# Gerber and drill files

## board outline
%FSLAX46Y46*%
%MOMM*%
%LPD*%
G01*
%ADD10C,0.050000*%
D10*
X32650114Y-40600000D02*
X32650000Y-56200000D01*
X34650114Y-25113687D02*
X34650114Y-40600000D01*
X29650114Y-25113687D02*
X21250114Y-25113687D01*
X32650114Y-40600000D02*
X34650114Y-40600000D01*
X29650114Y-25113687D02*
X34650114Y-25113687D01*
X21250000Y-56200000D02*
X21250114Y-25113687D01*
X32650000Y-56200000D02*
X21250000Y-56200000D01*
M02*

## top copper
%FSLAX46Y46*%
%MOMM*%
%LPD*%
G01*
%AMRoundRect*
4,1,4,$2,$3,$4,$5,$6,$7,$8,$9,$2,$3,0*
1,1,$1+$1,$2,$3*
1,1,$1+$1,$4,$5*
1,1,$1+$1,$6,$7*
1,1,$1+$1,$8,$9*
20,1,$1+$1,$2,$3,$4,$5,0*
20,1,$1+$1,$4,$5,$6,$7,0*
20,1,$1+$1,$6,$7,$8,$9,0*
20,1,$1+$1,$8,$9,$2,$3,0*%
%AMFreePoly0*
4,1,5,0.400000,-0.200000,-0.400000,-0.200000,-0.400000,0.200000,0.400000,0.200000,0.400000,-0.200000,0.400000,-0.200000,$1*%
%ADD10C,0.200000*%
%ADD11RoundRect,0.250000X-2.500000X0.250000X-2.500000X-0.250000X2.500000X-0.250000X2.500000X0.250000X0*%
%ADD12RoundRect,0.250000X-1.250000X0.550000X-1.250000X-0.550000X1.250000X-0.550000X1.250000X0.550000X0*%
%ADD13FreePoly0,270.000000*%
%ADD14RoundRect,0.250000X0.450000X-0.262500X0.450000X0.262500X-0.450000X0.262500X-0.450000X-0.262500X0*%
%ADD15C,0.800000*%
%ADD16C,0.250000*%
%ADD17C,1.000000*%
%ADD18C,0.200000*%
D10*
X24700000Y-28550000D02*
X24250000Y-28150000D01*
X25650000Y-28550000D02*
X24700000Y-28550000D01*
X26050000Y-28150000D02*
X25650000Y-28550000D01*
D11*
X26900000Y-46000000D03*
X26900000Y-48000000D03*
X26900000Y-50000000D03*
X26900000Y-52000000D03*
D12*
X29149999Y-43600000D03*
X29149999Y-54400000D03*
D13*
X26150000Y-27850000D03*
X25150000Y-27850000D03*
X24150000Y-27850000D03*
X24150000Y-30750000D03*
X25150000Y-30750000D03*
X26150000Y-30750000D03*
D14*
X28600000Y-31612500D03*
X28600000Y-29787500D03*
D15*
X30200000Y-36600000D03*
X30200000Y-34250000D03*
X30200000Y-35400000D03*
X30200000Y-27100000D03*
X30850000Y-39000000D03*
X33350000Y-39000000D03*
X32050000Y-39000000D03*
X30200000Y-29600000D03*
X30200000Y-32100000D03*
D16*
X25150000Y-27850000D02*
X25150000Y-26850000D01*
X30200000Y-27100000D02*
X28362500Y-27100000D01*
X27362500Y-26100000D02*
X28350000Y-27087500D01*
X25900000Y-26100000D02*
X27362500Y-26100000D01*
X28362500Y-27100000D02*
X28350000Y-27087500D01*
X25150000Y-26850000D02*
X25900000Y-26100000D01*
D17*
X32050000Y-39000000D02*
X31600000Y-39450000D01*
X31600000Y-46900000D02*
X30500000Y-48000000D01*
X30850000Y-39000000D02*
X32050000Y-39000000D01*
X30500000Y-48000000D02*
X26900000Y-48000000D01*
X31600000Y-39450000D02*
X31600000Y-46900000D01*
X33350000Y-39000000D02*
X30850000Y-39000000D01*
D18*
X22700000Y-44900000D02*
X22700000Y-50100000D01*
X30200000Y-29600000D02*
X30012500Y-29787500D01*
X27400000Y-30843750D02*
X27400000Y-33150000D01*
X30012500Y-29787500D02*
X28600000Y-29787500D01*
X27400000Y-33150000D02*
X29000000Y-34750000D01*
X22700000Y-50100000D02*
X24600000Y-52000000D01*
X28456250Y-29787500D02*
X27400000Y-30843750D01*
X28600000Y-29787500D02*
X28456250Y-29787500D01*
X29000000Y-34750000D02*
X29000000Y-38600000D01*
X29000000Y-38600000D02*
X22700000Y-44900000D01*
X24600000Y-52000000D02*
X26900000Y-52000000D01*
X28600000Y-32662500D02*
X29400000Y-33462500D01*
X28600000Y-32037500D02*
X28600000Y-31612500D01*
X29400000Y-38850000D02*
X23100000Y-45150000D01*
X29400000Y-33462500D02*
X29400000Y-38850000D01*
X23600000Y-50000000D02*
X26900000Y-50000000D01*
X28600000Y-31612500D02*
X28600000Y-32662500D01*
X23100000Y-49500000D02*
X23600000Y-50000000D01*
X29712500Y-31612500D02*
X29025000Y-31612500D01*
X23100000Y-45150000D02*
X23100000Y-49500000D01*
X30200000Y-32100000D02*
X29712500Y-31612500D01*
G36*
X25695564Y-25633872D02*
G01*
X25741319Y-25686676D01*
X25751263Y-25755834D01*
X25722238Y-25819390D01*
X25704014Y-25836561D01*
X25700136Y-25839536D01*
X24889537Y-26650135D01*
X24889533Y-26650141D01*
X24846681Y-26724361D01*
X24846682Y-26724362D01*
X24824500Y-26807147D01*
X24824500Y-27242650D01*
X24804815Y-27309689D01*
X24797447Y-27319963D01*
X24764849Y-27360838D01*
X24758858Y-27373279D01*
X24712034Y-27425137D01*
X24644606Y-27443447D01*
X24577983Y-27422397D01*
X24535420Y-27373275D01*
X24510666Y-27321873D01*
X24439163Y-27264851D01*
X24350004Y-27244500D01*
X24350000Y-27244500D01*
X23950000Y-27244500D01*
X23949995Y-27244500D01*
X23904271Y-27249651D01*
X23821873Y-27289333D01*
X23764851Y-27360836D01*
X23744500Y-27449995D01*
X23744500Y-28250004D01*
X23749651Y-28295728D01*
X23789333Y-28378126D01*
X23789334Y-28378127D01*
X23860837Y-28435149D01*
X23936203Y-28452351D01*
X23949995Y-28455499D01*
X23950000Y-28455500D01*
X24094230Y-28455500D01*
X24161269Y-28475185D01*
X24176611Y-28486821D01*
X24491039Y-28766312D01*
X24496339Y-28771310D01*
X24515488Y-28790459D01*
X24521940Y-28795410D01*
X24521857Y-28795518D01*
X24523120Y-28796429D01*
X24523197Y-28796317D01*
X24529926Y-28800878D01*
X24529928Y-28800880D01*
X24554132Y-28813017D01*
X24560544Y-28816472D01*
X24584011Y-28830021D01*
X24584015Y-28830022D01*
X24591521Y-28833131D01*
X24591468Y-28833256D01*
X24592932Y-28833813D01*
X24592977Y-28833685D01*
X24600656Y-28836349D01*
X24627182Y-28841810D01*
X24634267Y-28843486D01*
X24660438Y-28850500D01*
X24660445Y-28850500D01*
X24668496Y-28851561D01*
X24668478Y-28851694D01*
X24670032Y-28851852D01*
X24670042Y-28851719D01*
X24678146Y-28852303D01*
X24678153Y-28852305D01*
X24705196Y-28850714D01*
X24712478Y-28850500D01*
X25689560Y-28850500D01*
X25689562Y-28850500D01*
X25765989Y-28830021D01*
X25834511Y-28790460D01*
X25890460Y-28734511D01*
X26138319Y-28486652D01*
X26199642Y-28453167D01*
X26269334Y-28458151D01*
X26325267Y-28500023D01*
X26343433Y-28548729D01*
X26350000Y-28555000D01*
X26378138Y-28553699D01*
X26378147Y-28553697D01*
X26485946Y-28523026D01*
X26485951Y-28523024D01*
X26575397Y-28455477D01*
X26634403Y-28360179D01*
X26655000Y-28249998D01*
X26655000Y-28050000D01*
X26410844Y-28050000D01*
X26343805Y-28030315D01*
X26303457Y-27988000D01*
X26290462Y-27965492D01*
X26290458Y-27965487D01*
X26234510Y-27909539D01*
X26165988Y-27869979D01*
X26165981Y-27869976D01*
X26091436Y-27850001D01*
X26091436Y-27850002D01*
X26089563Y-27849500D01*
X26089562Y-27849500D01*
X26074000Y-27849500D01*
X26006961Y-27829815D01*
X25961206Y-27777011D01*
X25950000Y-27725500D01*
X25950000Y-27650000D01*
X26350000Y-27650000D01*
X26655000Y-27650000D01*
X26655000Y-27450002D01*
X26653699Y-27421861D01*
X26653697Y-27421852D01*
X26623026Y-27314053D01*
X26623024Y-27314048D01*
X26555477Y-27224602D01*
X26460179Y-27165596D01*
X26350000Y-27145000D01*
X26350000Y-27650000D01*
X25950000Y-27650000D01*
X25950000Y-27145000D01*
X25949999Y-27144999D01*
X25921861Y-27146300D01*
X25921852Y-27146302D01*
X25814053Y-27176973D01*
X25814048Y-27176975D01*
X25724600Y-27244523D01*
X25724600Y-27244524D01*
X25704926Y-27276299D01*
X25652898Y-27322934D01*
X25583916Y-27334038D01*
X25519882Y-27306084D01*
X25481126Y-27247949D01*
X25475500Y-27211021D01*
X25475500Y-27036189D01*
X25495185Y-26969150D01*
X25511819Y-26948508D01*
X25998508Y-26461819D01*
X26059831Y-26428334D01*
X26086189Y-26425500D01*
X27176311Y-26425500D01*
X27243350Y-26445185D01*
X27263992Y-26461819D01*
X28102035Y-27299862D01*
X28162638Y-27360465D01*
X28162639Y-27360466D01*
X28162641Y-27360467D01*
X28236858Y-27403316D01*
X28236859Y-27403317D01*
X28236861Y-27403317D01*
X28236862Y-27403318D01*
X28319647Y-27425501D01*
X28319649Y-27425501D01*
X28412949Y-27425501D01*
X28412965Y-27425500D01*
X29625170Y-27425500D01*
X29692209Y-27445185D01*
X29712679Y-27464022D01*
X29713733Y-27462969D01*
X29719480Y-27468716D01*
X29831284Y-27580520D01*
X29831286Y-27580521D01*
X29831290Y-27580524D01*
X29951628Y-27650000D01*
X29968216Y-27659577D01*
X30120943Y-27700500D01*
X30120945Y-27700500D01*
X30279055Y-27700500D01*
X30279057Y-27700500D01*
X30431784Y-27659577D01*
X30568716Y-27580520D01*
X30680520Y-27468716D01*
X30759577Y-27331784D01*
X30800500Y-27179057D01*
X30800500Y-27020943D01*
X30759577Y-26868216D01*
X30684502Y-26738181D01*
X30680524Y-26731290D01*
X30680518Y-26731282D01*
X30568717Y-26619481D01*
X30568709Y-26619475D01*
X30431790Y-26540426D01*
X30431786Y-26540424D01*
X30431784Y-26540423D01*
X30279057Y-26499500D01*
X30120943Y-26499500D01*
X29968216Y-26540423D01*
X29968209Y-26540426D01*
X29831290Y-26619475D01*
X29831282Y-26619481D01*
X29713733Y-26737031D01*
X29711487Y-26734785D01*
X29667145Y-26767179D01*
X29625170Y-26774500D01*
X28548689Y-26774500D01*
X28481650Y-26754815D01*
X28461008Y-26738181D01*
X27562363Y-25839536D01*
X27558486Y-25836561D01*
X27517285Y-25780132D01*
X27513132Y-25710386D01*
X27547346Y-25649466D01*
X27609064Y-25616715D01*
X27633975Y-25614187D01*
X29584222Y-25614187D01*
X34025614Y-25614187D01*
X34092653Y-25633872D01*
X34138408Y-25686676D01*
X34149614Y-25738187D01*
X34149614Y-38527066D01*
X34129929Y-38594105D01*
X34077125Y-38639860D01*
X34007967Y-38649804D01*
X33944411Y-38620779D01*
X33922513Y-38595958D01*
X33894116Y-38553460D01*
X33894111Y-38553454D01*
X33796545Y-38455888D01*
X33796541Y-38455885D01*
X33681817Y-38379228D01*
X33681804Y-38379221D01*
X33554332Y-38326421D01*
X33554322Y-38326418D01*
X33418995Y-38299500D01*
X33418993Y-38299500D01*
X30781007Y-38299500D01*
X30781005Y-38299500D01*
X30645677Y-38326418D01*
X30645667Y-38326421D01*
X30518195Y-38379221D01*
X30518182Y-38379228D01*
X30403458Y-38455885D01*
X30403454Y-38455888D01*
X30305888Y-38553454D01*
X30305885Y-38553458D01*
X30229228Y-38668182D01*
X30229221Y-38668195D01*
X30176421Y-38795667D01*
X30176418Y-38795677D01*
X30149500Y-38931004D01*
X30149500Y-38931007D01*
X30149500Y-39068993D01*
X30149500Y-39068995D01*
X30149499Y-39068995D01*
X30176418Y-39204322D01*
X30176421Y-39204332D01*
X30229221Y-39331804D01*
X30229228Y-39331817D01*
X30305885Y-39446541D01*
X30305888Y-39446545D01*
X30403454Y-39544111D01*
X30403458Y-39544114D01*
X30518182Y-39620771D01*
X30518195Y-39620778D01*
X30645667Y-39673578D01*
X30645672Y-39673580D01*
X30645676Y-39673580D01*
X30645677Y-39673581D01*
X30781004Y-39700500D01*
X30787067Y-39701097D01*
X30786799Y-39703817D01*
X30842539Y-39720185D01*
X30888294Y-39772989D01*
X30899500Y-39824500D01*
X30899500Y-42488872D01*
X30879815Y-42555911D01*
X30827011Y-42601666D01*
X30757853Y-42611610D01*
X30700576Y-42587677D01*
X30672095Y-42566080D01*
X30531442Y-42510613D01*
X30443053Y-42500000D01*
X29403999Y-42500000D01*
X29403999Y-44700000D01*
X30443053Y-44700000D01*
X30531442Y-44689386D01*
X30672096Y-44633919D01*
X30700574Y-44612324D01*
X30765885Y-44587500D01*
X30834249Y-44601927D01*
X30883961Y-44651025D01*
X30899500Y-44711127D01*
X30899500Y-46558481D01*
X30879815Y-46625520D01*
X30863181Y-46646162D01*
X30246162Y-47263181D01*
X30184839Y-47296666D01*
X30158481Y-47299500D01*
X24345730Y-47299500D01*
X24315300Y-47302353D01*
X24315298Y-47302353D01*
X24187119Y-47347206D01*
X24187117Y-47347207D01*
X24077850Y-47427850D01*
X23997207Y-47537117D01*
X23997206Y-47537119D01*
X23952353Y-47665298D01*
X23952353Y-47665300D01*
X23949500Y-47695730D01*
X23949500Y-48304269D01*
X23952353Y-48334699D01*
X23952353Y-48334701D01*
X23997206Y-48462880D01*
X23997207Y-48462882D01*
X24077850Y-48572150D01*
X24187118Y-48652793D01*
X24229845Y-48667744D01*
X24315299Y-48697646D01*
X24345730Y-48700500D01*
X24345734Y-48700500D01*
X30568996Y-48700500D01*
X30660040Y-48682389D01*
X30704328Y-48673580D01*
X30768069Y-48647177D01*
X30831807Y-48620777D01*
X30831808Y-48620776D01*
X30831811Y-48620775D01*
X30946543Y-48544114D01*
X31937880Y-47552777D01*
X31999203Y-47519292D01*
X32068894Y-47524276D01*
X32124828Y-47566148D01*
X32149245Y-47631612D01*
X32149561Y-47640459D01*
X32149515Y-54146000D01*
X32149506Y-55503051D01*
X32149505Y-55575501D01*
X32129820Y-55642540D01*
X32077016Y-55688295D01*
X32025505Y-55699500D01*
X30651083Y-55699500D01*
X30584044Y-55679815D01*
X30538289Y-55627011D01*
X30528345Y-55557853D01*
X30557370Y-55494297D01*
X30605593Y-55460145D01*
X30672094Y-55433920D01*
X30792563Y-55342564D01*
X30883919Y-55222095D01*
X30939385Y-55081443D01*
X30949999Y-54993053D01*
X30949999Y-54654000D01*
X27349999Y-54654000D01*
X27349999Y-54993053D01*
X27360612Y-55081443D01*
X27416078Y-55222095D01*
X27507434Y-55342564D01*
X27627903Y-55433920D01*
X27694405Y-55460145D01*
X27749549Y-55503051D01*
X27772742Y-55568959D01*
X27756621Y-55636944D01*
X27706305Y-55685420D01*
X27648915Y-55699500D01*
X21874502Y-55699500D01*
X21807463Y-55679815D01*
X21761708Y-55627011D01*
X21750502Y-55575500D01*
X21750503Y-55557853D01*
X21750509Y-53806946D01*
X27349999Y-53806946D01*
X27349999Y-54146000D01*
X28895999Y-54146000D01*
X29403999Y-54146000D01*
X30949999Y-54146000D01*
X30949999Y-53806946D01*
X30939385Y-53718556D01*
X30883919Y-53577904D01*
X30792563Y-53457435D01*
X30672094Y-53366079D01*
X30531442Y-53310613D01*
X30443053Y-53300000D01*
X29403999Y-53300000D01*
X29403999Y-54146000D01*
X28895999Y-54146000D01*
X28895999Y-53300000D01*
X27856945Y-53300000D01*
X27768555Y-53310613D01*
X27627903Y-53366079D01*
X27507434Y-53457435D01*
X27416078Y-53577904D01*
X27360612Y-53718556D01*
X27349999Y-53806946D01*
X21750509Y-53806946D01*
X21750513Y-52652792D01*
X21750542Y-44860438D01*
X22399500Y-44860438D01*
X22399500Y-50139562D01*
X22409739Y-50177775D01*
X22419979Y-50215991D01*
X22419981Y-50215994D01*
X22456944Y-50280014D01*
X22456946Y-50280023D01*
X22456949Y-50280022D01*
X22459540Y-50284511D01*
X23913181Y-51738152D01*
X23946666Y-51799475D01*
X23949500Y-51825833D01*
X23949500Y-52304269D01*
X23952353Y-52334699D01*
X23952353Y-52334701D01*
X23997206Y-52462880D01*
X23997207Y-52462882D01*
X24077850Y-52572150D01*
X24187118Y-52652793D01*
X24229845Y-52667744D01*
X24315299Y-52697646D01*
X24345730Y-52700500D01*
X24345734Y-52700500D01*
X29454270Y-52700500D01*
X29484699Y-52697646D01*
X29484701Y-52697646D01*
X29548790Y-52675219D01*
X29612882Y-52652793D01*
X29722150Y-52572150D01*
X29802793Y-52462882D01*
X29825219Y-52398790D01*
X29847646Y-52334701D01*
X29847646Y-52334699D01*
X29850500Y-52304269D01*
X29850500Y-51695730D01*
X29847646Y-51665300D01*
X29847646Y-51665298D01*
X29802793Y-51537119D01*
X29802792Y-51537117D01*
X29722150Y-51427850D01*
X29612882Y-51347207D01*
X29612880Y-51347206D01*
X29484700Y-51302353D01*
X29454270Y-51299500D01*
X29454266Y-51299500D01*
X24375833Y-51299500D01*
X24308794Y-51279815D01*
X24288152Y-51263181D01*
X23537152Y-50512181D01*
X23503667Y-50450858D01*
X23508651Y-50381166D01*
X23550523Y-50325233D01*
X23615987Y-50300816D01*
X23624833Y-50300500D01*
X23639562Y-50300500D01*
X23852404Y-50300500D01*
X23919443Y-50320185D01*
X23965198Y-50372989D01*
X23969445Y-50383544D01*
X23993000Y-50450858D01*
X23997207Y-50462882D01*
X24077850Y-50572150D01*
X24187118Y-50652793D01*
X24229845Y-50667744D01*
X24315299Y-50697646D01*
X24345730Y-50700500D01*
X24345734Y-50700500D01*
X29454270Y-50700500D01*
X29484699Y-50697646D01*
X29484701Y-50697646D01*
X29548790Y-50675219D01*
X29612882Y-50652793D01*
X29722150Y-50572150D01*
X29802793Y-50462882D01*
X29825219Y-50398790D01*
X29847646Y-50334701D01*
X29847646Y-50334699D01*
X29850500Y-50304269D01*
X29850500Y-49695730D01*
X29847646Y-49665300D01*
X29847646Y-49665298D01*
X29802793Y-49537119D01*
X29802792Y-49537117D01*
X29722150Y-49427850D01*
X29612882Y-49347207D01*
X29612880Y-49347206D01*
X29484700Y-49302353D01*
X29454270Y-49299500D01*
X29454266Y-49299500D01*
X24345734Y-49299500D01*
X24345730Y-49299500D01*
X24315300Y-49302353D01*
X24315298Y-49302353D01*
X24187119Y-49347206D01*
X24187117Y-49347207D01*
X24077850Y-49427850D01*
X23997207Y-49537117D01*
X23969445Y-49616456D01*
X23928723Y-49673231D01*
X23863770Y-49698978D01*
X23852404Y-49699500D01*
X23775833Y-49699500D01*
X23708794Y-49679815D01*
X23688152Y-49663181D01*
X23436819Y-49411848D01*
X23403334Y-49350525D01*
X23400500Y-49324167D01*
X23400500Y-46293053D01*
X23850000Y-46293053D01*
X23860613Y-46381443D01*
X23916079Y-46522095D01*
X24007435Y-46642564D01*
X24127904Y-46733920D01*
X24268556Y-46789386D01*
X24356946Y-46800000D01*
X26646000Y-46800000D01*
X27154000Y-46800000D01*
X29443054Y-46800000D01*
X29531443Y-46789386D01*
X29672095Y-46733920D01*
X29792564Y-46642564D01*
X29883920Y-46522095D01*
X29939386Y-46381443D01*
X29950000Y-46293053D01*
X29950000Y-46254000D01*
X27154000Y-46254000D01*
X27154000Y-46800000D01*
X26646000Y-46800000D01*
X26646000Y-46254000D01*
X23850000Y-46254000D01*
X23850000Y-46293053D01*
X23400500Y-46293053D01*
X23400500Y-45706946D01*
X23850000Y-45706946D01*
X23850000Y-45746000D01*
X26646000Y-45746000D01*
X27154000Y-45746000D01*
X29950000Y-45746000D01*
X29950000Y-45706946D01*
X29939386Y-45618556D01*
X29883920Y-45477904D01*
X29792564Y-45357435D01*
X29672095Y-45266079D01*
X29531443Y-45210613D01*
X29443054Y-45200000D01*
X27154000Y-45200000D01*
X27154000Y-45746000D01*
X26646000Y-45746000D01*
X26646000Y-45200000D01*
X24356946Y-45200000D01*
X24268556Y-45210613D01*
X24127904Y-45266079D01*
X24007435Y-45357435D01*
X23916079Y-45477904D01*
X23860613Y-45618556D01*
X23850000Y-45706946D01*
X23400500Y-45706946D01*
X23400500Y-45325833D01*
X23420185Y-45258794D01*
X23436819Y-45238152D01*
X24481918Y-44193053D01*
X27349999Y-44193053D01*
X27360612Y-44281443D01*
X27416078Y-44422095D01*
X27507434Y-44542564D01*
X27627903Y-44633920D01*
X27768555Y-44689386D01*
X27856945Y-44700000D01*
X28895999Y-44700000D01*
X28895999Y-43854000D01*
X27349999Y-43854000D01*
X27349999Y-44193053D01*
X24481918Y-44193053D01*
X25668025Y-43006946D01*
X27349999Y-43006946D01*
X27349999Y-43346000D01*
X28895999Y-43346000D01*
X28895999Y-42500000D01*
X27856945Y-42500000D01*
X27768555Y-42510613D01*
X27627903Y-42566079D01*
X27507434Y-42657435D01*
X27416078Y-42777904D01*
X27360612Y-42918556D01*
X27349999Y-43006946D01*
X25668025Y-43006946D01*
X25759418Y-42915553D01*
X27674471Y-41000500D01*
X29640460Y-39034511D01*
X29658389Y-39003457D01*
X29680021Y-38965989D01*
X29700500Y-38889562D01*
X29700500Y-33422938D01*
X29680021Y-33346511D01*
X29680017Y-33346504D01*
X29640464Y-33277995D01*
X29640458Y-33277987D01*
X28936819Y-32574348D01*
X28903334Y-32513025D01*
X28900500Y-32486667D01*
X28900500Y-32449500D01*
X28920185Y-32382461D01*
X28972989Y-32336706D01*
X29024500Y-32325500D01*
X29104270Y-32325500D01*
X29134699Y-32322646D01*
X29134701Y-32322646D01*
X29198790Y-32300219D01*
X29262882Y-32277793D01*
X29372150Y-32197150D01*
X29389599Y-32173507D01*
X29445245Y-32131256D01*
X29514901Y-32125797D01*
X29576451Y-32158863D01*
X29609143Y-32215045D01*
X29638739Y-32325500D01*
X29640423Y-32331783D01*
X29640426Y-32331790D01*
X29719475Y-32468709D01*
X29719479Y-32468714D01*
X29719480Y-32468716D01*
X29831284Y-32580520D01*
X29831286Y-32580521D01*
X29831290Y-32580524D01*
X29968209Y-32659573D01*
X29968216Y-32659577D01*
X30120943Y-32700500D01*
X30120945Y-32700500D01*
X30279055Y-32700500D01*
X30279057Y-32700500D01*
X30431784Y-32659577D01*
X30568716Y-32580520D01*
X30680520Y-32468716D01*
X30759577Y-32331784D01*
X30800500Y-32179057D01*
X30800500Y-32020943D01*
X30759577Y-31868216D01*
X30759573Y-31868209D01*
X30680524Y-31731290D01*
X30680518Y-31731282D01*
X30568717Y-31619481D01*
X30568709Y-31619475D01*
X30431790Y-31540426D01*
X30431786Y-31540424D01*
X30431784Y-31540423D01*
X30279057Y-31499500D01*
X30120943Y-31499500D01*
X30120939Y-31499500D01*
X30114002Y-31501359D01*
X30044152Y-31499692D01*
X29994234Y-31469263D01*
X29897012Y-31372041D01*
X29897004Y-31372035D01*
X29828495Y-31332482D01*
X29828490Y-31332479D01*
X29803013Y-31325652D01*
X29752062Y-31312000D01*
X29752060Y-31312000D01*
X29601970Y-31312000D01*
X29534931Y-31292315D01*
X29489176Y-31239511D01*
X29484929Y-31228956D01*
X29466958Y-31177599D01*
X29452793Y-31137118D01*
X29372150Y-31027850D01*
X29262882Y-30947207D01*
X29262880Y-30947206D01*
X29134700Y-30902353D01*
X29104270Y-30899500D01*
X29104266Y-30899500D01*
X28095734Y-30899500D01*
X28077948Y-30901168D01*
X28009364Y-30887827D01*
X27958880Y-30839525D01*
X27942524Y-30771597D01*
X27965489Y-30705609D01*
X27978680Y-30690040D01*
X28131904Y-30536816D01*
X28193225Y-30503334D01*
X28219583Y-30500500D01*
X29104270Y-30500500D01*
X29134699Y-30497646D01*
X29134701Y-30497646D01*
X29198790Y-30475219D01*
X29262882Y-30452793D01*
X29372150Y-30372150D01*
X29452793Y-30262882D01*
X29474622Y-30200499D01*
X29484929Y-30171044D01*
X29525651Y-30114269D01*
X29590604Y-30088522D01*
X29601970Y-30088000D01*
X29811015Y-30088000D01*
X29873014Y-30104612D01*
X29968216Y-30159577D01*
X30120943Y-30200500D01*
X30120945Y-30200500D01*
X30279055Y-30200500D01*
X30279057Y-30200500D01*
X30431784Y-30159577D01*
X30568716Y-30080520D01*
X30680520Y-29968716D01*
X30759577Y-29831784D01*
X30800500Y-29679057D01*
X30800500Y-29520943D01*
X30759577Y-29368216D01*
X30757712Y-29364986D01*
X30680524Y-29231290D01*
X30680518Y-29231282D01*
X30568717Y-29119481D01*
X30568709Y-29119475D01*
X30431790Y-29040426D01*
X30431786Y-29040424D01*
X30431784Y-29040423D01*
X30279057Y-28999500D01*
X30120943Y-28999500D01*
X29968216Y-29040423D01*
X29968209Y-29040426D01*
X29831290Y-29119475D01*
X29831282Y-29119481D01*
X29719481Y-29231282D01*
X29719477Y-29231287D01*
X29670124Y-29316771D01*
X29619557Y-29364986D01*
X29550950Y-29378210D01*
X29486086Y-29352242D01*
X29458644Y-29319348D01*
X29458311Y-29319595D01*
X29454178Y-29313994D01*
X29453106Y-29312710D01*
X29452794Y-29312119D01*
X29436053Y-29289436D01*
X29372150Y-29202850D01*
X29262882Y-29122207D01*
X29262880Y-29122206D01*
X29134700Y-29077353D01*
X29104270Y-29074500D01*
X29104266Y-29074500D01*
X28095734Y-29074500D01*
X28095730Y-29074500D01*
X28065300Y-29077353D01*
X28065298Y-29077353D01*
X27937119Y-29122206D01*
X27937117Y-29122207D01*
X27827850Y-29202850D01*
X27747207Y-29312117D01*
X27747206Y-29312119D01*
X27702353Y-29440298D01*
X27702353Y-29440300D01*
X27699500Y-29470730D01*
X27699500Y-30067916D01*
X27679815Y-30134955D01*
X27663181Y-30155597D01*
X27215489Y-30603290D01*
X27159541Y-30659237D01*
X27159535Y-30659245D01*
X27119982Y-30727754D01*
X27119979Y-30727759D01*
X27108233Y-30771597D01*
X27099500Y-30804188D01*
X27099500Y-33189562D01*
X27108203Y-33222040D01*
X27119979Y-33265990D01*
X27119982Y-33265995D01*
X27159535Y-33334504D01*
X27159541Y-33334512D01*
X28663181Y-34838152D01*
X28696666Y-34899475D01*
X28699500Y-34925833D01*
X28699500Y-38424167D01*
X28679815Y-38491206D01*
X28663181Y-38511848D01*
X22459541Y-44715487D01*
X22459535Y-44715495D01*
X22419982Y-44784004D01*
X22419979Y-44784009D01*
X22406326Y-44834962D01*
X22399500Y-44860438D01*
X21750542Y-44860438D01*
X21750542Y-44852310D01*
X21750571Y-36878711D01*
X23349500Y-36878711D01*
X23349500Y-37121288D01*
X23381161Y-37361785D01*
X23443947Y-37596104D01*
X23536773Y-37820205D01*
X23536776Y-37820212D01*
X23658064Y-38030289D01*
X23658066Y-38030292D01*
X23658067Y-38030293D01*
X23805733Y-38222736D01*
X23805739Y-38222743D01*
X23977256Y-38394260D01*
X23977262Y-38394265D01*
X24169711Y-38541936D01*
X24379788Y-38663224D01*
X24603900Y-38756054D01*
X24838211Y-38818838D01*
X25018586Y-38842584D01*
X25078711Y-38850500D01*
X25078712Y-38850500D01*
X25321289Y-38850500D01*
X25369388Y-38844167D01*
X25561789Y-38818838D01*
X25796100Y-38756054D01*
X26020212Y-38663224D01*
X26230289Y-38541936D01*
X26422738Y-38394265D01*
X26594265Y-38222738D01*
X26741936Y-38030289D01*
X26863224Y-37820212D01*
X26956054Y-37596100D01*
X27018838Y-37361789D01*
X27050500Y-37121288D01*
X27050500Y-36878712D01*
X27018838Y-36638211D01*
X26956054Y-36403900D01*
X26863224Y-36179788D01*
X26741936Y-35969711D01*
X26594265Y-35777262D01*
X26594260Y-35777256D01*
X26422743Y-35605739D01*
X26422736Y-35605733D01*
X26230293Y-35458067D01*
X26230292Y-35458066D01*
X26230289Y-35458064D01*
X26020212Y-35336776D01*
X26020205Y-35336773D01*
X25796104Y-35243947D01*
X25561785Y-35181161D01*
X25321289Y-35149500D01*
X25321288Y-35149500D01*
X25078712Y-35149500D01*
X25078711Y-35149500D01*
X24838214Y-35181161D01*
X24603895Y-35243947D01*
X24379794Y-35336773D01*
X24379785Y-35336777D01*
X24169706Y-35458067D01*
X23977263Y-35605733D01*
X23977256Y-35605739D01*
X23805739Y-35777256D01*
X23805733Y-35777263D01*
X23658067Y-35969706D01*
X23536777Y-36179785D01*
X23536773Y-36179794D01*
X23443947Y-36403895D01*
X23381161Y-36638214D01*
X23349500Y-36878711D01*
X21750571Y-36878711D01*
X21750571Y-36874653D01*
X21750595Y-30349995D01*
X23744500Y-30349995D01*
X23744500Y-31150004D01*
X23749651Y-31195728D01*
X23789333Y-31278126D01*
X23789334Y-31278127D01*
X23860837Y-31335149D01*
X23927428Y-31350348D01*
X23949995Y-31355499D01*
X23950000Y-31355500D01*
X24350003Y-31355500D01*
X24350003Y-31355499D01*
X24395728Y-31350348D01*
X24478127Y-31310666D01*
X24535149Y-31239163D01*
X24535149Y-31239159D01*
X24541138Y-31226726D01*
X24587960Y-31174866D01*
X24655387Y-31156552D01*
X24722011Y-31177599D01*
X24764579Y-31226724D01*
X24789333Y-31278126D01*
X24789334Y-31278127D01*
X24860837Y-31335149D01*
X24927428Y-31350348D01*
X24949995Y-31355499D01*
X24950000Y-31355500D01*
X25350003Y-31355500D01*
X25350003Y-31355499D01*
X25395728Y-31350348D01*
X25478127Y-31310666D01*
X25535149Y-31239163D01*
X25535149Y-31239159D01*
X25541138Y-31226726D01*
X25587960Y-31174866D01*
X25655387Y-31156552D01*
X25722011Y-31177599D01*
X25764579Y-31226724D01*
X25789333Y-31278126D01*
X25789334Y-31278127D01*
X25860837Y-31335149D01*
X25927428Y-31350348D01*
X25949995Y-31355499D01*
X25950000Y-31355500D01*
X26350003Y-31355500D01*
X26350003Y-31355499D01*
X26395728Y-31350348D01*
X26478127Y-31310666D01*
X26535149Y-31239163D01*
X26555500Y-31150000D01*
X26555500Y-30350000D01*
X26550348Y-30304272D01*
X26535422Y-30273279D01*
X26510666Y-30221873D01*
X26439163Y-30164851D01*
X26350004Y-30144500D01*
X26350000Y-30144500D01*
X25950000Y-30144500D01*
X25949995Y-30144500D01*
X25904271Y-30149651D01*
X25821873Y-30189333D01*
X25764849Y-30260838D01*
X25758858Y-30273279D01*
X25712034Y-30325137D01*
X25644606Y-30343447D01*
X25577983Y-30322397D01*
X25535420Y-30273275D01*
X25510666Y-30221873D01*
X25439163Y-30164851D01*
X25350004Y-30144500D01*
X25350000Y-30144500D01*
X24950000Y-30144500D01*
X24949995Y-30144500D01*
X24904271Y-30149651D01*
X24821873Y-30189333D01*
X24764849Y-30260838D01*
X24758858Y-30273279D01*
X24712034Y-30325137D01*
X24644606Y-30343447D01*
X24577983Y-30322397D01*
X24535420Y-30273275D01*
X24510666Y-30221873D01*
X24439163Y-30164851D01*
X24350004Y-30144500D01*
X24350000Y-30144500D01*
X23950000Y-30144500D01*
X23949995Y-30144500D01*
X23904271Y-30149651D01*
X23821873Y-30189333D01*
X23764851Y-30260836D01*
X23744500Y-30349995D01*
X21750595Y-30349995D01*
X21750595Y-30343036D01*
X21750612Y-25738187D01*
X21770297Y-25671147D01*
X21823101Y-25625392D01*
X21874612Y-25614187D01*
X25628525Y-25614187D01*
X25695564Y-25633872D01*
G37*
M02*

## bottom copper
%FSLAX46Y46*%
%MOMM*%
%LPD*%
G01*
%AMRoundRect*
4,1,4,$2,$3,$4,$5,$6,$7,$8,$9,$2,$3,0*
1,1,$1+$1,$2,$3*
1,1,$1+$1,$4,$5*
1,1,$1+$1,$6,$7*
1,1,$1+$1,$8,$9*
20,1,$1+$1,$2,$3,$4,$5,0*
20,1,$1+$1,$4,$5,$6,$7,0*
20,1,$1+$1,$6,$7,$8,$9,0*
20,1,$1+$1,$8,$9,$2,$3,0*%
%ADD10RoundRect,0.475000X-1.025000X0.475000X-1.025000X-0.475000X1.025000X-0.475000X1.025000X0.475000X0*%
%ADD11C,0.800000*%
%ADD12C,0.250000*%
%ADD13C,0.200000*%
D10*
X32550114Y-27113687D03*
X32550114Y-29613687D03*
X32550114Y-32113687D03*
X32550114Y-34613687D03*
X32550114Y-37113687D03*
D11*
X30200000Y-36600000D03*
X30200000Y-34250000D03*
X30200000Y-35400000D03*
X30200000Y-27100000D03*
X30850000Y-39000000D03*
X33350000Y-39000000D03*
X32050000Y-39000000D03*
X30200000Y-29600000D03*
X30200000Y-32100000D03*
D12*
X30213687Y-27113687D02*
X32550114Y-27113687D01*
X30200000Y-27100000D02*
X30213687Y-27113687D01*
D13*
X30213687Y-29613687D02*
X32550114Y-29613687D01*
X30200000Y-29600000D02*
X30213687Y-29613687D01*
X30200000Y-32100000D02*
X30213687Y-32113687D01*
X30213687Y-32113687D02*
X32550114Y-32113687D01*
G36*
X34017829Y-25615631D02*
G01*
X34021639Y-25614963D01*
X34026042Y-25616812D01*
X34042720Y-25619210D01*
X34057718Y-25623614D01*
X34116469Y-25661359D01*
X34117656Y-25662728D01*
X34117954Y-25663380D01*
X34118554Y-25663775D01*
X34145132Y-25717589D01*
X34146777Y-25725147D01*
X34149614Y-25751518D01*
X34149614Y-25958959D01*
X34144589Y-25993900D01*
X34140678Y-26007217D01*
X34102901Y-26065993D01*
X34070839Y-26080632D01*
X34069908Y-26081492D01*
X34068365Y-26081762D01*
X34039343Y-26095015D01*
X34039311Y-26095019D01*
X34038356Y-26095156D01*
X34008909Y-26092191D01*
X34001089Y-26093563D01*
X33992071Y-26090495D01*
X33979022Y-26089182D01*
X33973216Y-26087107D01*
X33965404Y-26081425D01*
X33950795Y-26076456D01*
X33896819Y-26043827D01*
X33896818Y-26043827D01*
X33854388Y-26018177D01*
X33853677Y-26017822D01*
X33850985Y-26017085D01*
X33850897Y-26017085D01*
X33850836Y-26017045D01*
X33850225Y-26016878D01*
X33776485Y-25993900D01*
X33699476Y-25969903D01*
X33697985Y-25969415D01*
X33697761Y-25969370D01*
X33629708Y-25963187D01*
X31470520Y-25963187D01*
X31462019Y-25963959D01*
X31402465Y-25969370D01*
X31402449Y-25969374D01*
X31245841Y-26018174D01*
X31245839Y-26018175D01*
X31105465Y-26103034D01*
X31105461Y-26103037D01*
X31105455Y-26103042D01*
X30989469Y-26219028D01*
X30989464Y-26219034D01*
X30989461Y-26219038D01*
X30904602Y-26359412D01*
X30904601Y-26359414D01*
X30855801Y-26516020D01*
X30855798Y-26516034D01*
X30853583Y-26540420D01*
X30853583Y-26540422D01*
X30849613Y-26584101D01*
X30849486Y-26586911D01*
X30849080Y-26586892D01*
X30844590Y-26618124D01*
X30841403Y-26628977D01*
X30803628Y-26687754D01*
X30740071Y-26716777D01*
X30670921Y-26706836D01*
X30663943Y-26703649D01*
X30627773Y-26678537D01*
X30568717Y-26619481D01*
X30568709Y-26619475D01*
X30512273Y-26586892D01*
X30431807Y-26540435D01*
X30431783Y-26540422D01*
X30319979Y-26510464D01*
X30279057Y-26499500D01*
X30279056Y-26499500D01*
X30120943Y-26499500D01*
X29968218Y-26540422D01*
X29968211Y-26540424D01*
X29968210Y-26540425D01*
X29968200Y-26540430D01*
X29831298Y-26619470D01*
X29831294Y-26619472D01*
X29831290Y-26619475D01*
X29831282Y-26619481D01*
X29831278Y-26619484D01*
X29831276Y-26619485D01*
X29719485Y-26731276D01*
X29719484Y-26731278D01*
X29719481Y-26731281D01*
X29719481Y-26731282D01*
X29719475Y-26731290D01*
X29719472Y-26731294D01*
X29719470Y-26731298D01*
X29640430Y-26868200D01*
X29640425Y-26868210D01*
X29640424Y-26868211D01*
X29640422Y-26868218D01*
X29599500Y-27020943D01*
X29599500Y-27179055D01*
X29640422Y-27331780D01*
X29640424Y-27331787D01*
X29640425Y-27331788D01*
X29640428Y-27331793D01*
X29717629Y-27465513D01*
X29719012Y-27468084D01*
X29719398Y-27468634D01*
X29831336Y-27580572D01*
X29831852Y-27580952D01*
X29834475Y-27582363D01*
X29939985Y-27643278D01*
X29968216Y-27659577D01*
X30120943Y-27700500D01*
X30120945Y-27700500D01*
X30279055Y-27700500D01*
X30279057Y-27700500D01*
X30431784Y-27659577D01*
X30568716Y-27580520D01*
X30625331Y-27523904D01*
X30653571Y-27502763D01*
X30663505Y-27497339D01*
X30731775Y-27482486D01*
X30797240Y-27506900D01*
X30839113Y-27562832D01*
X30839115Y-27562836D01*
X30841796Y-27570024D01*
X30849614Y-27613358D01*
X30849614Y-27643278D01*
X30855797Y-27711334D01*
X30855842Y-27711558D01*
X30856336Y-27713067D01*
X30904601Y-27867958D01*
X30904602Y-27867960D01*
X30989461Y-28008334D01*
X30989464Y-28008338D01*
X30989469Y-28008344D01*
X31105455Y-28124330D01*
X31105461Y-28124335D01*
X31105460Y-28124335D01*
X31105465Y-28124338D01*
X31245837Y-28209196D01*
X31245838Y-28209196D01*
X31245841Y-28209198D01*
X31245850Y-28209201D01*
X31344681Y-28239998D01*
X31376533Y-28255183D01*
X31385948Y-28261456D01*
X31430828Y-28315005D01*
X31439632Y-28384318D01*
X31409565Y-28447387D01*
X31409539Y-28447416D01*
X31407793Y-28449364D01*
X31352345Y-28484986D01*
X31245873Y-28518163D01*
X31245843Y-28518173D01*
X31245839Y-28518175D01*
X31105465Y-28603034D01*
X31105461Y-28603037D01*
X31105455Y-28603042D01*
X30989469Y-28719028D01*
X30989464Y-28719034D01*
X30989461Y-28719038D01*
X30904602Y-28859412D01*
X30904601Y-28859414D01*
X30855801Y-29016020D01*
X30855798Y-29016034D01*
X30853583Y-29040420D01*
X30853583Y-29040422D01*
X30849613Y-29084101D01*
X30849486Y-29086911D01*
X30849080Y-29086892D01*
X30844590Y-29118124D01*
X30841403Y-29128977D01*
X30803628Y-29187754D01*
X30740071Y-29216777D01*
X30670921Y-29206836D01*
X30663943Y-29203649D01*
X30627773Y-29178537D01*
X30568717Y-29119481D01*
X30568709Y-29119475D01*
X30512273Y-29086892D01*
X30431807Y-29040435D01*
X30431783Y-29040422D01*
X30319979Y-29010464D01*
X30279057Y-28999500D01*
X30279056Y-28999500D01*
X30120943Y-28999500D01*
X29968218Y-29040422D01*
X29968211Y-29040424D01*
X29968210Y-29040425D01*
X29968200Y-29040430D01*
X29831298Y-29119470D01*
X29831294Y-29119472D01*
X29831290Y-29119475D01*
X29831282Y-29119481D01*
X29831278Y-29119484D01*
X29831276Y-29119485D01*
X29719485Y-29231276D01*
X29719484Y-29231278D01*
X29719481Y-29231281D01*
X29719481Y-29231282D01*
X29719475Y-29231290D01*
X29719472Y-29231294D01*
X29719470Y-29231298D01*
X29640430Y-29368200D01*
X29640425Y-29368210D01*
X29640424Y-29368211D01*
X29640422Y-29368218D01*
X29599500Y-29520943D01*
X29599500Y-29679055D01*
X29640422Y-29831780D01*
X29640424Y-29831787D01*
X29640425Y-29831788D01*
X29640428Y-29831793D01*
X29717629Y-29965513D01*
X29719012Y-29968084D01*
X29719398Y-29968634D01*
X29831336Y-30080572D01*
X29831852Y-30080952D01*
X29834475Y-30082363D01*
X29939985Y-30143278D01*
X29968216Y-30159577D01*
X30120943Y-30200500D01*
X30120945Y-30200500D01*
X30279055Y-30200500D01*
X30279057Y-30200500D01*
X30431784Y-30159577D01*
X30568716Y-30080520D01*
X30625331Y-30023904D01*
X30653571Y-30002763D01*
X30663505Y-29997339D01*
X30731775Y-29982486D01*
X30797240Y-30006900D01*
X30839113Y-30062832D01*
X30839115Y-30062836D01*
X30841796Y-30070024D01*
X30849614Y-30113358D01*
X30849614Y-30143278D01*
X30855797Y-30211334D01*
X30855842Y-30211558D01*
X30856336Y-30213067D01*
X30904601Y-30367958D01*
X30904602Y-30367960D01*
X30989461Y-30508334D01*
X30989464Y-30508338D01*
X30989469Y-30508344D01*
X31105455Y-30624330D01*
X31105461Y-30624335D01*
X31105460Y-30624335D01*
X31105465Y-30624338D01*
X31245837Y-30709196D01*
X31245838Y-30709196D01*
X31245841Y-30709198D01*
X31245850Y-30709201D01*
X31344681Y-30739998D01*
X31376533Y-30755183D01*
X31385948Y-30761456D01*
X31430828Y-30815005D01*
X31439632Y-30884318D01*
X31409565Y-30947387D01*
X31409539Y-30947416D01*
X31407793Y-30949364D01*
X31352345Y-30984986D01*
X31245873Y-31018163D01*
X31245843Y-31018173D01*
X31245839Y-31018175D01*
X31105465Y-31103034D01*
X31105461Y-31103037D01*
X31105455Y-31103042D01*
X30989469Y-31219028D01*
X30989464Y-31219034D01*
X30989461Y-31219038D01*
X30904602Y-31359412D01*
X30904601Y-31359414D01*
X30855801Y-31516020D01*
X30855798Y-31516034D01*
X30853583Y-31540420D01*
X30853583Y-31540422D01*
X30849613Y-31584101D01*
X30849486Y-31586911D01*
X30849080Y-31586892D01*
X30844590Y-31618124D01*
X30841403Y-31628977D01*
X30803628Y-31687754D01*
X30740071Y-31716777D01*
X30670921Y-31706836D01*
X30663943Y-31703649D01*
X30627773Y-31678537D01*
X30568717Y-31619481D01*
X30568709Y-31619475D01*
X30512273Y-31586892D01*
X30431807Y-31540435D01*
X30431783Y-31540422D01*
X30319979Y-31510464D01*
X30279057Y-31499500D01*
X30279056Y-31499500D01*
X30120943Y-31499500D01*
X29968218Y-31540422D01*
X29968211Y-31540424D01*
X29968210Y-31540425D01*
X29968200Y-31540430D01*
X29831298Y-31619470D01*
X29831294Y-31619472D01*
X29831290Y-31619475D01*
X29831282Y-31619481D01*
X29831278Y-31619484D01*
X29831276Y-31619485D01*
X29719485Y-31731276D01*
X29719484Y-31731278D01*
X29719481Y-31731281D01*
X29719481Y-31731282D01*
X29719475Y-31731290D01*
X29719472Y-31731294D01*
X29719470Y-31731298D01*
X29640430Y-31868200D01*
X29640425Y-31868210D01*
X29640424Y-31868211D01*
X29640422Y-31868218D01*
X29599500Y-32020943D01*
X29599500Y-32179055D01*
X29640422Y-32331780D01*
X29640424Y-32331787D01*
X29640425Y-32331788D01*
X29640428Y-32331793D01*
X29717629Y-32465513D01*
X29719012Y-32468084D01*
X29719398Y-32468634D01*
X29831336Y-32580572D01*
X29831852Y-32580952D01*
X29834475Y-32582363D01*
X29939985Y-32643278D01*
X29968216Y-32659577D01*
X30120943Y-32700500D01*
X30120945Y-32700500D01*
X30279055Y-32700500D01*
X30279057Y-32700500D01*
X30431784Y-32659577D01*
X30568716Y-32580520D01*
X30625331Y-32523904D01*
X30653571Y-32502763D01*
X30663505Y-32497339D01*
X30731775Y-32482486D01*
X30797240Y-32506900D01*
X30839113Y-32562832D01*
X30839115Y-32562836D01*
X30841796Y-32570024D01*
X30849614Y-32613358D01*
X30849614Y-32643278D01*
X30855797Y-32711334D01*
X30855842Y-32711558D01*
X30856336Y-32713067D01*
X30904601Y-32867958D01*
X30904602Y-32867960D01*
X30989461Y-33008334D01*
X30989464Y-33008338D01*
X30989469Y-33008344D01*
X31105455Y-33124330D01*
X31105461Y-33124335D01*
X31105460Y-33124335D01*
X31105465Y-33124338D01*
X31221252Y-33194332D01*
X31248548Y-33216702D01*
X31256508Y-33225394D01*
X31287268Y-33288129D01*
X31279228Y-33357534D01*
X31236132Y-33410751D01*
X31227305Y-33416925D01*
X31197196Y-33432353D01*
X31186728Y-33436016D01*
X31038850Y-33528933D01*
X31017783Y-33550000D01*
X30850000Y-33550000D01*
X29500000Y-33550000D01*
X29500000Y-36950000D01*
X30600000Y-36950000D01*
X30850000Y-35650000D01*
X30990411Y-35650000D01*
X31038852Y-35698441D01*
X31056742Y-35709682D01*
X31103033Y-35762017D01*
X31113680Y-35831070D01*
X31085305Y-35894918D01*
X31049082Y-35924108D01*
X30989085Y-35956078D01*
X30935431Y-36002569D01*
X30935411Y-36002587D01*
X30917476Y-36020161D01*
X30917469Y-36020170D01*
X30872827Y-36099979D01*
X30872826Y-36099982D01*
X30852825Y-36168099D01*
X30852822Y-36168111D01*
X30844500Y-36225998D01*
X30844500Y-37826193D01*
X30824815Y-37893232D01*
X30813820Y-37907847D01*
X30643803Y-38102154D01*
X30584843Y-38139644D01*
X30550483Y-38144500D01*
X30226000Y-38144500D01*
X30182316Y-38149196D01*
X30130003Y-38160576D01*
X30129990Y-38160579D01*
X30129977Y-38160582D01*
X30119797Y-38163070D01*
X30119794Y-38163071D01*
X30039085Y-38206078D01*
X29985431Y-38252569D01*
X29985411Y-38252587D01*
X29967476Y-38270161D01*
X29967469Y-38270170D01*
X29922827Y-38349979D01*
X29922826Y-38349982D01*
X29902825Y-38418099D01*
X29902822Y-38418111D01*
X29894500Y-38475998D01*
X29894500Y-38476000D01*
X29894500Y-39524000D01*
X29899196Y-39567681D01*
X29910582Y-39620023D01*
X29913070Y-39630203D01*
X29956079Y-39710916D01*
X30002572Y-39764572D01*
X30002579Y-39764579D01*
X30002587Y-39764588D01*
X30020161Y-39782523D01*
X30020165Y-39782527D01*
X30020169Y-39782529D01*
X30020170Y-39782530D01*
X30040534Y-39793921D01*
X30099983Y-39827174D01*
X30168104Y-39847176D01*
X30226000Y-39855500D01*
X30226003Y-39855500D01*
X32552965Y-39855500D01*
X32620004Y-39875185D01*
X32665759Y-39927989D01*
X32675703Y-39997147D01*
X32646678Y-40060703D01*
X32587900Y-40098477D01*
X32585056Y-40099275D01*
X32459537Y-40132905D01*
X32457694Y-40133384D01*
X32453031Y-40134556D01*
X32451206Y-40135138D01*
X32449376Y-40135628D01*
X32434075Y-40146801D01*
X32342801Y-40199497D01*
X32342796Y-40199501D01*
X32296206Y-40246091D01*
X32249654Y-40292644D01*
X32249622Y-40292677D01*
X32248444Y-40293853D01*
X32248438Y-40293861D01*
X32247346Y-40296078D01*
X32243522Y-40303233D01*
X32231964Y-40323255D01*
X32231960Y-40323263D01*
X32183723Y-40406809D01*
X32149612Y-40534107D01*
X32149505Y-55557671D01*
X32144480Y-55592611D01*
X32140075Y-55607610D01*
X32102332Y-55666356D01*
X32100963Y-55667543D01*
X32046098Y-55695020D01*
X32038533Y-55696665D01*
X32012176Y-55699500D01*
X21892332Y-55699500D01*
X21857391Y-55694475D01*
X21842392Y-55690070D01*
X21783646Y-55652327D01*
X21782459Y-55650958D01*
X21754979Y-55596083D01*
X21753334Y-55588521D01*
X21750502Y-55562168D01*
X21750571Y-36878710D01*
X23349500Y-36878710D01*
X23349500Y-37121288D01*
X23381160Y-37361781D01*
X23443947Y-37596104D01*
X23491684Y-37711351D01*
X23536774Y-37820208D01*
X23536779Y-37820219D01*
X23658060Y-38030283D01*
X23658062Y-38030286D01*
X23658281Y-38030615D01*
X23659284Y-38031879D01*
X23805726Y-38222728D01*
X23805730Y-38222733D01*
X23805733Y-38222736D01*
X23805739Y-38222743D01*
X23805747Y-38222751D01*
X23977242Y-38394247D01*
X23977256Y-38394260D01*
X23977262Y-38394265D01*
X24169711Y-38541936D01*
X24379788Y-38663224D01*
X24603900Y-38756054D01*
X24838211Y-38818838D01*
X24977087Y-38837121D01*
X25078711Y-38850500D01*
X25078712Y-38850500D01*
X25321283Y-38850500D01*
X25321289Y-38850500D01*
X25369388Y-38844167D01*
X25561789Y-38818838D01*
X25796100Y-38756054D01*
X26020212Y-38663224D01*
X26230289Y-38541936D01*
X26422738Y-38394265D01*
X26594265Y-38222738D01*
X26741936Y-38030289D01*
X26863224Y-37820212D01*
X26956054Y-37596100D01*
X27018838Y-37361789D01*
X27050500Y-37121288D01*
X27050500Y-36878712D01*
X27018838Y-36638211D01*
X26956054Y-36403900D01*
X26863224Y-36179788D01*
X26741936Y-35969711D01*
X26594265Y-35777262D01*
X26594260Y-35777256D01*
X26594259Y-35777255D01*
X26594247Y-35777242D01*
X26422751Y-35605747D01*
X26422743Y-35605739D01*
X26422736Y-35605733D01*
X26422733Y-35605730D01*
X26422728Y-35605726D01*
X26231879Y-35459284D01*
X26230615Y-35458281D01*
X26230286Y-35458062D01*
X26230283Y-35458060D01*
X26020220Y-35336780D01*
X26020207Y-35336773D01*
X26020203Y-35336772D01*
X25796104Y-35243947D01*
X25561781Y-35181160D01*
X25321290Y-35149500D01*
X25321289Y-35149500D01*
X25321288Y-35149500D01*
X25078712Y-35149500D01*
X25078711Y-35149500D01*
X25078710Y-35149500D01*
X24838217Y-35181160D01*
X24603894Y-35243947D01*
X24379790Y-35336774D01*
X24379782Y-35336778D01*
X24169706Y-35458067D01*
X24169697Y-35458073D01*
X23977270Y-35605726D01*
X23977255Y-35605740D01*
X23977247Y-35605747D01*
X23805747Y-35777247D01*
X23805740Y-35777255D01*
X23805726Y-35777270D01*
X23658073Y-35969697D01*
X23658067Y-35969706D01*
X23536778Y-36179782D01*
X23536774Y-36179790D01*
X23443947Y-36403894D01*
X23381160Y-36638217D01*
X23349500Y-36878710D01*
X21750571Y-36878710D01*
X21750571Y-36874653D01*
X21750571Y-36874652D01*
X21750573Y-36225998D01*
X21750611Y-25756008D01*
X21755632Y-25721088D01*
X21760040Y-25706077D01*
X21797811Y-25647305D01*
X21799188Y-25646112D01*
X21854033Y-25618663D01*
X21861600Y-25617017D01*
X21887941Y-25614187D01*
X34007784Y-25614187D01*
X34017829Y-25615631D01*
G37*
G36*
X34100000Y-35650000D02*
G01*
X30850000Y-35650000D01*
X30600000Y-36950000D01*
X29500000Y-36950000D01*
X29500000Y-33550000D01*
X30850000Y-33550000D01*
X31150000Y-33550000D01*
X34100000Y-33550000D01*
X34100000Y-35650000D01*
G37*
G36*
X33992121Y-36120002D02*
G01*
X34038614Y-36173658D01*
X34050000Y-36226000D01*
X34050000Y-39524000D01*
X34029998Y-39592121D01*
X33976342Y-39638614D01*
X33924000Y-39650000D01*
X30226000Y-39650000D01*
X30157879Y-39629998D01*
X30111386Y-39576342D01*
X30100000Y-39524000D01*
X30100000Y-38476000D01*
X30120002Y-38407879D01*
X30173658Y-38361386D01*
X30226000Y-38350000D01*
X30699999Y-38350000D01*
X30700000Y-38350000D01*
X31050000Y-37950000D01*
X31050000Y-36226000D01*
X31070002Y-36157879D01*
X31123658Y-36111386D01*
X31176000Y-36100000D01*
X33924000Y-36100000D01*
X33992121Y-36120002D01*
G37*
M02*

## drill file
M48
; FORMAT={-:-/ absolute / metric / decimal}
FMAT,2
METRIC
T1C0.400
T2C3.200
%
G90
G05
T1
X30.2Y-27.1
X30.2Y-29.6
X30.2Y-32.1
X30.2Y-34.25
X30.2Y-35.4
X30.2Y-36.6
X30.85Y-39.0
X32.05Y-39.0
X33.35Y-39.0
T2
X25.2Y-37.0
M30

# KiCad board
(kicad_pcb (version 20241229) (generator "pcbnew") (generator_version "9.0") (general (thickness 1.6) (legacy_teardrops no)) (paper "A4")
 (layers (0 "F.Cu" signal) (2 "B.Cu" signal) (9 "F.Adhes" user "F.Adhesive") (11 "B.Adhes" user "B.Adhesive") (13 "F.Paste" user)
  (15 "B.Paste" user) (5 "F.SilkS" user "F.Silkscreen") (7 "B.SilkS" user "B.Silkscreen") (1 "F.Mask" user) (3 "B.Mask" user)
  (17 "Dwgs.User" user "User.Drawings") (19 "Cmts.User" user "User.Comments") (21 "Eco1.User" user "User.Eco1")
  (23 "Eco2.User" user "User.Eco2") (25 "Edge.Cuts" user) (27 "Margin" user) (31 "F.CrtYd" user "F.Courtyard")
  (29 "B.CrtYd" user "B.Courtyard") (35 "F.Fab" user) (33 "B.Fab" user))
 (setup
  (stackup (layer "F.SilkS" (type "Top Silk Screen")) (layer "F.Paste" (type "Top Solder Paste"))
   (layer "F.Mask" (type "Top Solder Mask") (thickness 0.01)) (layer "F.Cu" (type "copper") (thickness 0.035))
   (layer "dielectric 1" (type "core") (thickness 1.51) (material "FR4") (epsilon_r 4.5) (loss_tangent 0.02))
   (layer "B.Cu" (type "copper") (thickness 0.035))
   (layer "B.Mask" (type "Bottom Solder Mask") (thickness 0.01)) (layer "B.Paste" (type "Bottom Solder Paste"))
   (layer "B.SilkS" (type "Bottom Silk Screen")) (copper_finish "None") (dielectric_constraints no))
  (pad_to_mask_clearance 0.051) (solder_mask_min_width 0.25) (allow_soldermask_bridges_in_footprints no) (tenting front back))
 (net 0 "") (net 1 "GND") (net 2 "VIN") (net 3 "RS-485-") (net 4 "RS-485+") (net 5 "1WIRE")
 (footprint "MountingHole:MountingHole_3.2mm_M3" (layer "F.Cu") (at 25.2 37)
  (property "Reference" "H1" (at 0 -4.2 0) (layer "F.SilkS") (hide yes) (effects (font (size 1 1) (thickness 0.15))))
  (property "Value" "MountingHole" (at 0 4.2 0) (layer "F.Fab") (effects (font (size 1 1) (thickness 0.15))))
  (pad "" np_thru_hole circle (at 0 0) (size 3.2 3.2) (drill 3.2) (layers "*.Cu" "*.Mask")))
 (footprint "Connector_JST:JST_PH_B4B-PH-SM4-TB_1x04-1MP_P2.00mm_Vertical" (layer "F.Cu") (at 27.4 49 -90)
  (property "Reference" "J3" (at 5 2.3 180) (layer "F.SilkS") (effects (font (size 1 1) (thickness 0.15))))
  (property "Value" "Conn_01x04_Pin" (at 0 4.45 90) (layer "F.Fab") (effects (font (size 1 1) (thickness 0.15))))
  (pad "1" smd roundrect (at -3 0.5 270) (size 1 5.5) (layers "F.Cu" "F.Mask" "F.Paste") (roundrect_rratio 0.25) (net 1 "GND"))
  (pad "2" smd roundrect (at -1 0.5 270) (size 1 5.5) (layers "F.Cu" "F.Mask" "F.Paste") (roundrect_rratio 0.25) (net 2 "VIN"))
  (pad "3" smd roundrect (at 1 0.5 270) (size 1 5.5) (layers "F.Cu" "F.Mask" "F.Paste") (roundrect_rratio 0.25) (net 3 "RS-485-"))
  (pad "4" smd roundrect (at 3 0.5 270) (size 1 5.5) (layers "F.Cu" "F.Mask" "F.Paste") (roundrect_rratio 0.25) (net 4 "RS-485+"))
  (pad "MP" smd roundrect (at -5.4 -1.749999 270) (size 1.6 3) (layers "F.Cu" "F.Mask" "F.Paste") (roundrect_rratio 0.15625) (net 1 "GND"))
  (pad "MP" smd roundrect (at 5.4 -1.749999 270) (size 1.6 3) (layers "F.Cu" "F.Mask" "F.Paste") (roundrect_rratio 0.15625) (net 1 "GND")))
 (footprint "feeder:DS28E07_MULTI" (layer "F.Cu") (at 25.15 29.3 -90)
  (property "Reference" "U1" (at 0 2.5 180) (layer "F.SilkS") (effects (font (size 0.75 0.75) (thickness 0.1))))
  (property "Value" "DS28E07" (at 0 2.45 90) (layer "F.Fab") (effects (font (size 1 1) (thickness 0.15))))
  (fp_line (start -0.75 0.45) (end -1.15 0.9) (stroke (width 0.2) (type solid)) (layer "F.Cu"))
  (fp_line (start -0.75 -0.5) (end -0.75 0.45) (stroke (width 0.2) (type solid)) (layer "F.Cu"))
  (fp_line (start -1.15 -0.9) (end -0.75 -0.5) (stroke (width 0.2) (type solid)) (layer "F.Cu"))
  (pad "1" smd custom (at -1.45 -1 270) (size 0.8 0.4) (layers "F.Cu" "F.Mask" "F.Paste") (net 1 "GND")
   (options (clearance outline) (anchor rect)) (primitives))
  (pad "2" smd custom (at -1.45 0 270) (size 0.8 0.4) (layers "F.Cu" "F.Mask" "F.Paste") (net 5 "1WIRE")
   (options (clearance outline) (anchor rect)) (primitives))
  (pad "3" smd custom (at -1.45 1 270) (size 0.8 0.4) (layers "F.Cu" "F.Mask" "F.Paste") (options (clearance outline) (anchor rect))
   (primitives))
  (pad "4" smd custom (at 1.45 1 270) (size 0.8 0.4) (layers "F.Cu" "F.Mask" "F.Paste") (options (clearance outline) (anchor rect))
   (primitives))
  (pad "5" smd custom (at 1.45 0 270) (size 0.8 0.4) (layers "F.Cu" "F.Mask" "F.Paste") (options (clearance outline) (anchor rect))
   (primitives))
  (pad "6" smd custom (at 1.45 -1 270) (size 0.8 0.4) (layers "F.Cu" "F.Mask" "F.Paste") (options (clearance outline) (anchor rect))
   (primitives)))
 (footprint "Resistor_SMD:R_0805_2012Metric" (layer "F.Cu") (at 28.6 30.7 90)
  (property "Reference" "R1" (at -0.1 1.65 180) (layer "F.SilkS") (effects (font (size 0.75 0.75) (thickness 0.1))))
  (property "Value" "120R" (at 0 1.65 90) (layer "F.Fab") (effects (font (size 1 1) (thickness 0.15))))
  (pad "1" smd roundrect (at -0.9125 0 90) (size 1.025 1.4) (layers "F.Cu" "F.Mask" "F.Paste") (roundrect_rratio 0.243902439)
   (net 3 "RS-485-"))
  (pad "2" smd roundrect (at 0.9125 0 90) (size 1.025 1.4) (layers "F.Cu" "F.Mask" "F.Paste") (roundrect_rratio 0.243902439)
   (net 4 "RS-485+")))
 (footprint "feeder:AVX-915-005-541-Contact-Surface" (layer "B.Cu") (at 32.550114 27.113687 -90)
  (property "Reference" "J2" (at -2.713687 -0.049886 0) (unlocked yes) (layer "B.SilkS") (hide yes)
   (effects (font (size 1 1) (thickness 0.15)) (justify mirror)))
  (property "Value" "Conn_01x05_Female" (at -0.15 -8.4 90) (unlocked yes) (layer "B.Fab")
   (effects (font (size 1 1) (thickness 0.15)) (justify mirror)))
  (pad "1" smd roundrect (at 0 0 270) (size 1.9 3) (layers "B.Cu" "B.Mask" "B.Paste") (roundrect_rratio 0.25) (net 5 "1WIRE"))
  (pad "2" smd roundrect (at 2.5 0 270) (size 1.9 3) (layers "B.Cu" "B.Mask" "B.Paste") (roundrect_rratio 0.25) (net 4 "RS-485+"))
  (pad "3" smd roundrect (at 5 0 270) (size 1.9 3) (layers "B.Cu" "B.Mask" "B.Paste") (roundrect_rratio 0.25) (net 3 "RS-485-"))
  (pad "4" smd roundrect (at 7.5 0 270) (size 1.9 3) (layers "B.Cu" "B.Mask" "B.Paste") (roundrect_rratio 0.25) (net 1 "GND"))
  (pad "5" smd roundrect (at 10 0 270) (size 1.9 3) (layers "B.Cu" "B.Mask" "B.Paste") (roundrect_rratio 0.25) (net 2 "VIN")))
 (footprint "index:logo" (layer "B.Cu") (at 26.95 48.8 180)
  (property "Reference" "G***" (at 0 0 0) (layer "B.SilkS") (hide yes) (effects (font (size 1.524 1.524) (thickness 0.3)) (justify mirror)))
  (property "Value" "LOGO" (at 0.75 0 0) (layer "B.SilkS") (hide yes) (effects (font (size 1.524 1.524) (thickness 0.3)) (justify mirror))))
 (gr_line (start 32.650114 40.6) (end 32.65 56.2) (stroke (width 0.05) (type solid)) (layer "Edge.Cuts"))
 (gr_line (start 34.650114 25.113687) (end 34.650114 40.6) (stroke (width 0.05) (type solid)) (layer "Edge.Cuts"))
 (gr_line (start 29.650114 25.113687) (end 21.250114 25.113687) (stroke (width 0.05) (type solid)) (layer "Edge.Cuts"))
 (gr_line (start 32.650114 40.6) (end 34.650114 40.6) (stroke (width 0.05) (type solid)) (layer "Edge.Cuts"))
 (gr_line (start 29.650114 25.113687) (end 34.650114 25.113687) (stroke (width 0.05) (type solid)) (layer "Edge.Cuts"))
 (gr_line (start 21.25 56.2) (end 21.250114 25.113687) (stroke (width 0.05) (type solid)) (layer "Edge.Cuts"))
 (gr_line (start 32.65 56.2) (end 21.25 56.2) (stroke (width 0.05) (type solid)) (layer "Edge.Cuts"))
 (via (at 30.2 36.6) (size 0.8) (drill 0.4) (layers "F.Cu" "B.Cu") (free yes) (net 1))
 (via (at 30.2 34.25) (size 0.8) (drill 0.4) (layers "F.Cu" "B.Cu") (free yes) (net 1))
 (via (at 30.2 35.4) (size 0.8) (drill 0.4) (layers "F.Cu" "B.Cu") (free yes) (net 1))
 (segment (start 25.15 27.85) (end 25.15 26.85) (width 0.25) (layer "F.Cu") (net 5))
 (segment (start 30.2 27.1) (end 28.3625 27.1) (width 0.25) (layer "F.Cu") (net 5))
 (segment (start 27.3625 26.1) (end 28.35 27.0875) (width 0.25) (layer "F.Cu") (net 5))
 (segment (start 25.9 26.1) (end 27.3625 26.1) (width 0.25) (layer "F.Cu") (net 5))
 (segment (start 28.3625 27.1) (end 28.35 27.0875) (width 0.25) (layer "F.Cu") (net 5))
 (segment (start 25.15 26.85) (end 25.9 26.1) (width 0.25) (layer "F.Cu") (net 5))
 (via (at 30.2 27.1) (size 0.8) (drill 0.4) (layers "F.Cu" "B.Cu") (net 5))
 (segment (start 30.213687 27.113687) (end 32.550114 27.113687) (width 0.25) (layer "B.Cu") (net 5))
 (segment (start 30.2 27.1) (end 30.213687 27.113687) (width 0.25) (layer "B.Cu") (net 5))
 (segment (start 32.05 39) (end 31.6 39.45) (width 1) (layer "F.Cu") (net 2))
 (segment (start 31.6 46.9) (end 30.5 48) (width 1) (layer "F.Cu") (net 2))
 (segment (start 30.85 39) (end 32.05 39) (width 1) (layer "F.Cu") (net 2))
 (segment (start 30.5 48) (end 26.9 48) (width 1) (layer "F.Cu") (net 2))
 (segment (start 31.6 39.45) (end 31.6 46.9) (width 1) (layer "F.Cu") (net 2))
 (segment (start 33.35 39) (end 30.85 39) (width 1) (layer "F.Cu") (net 2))
 (via (at 30.85 39) (size 0.8) (drill 0.4) (layers "F.Cu" "B.Cu") (free yes) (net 2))
 (via (at 33.35 39) (size 0.8) (drill 0.4) (layers "F.Cu" "B.Cu") (free yes) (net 2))
 (via (at 32.05 39) (size 0.8) (drill 0.4) (layers "F.Cu" "B.Cu") (free yes) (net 2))
 (segment (start 22.7 44.9) (end 22.7 50.1) (width 0.2) (layer "F.Cu") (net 4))
 (segment (start 30.2 29.6) (end 30.0125 29.7875) (width 0.2) (layer "F.Cu") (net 4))
 (segment (start 27.4 30.84375) (end 27.4 33.15) (width 0.2) (layer "F.Cu") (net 4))
 (segment (start 30.0125 29.7875) (end 28.6 29.7875) (width 0.2) (layer "F.Cu") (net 4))
 (segment (start 27.4 33.15) (end 29 34.75) (width 0.2) (layer "F.Cu") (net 4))
 (segment (start 22.7 50.1) (end 24.6 52) (width 0.2) (layer "F.Cu") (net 4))
 (segment (start 28.45625 29.7875) (end 27.4 30.84375) (width 0.2) (layer "F.Cu") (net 4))
 (segment (start 28.6 29.7875) (end 28.45625 29.7875) (width 0.2) (layer "F.Cu") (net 4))
 (segment (start 29 34.75) (end 29 38.6) (width 0.2) (layer "F.Cu") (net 4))
 (segment (start 29 38.6) (end 22.7 44.9) (width 0.2) (layer "F.Cu") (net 4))
 (segment (start 24.6 52) (end 26.9 52) (width 0.2) (layer "F.Cu") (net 4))
 (via (at 30.2 29.6) (size 0.8) (drill 0.4) (layers "F.Cu" "B.Cu") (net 4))
 (segment (start 30.213687 29.613687) (end 32.550114 29.613687) (width 0.2) (layer "B.Cu") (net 4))
 (segment (start 30.2 29.6) (end 30.213687 29.613687) (width 0.2) (layer "B.Cu") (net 4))
 (segment (start 28.6 32.6625) (end 29.4 33.4625) (width 0.2) (layer "F.Cu") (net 3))
 (segment (start 28.6 32.0375) (end 28.6 31.6125) (width 0.2) (layer "F.Cu") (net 3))
 (segment (start 29.4 38.85) (end 23.1 45.15) (width 0.2) (layer "F.Cu") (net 3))
 (segment (start 29.4 33.4625) (end 29.4 38.85) (width 0.2) (layer "F.Cu") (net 3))
 (segment (start 23.6 50) (end 26.9 50) (width 0.2) (layer "F.Cu") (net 3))
 (segment (start 28.6 31.6125) (end 28.6 32.6625) (width 0.2) (layer "F.Cu") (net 3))
 (segment (start 23.1 49.5) (end 23.6 50) (width 0.2) (layer "F.Cu") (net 3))
 (segment (start 29.7125 31.6125) (end 29.025 31.6125) (width 0.2) (layer "F.Cu") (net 3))
 (segment (start 23.1 45.15) (end 23.1 49.5) (width 0.2) (layer "F.Cu") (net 3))
 (segment (start 30.2 32.1) (end 29.7125 31.6125) (width 0.2) (layer "F.Cu") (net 3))
 (via (at 30.2 32.1) (size 0.8) (drill 0.4) (layers "F.Cu" "B.Cu") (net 3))
 (segment (start 30.2 32.1) (end 30.213687 32.113687) (width 0.2) (layer "B.Cu") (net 3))
 (segment (start 30.213687 32.113687) (end 32.550114 32.113687) (width 0.2) (layer "B.Cu") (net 3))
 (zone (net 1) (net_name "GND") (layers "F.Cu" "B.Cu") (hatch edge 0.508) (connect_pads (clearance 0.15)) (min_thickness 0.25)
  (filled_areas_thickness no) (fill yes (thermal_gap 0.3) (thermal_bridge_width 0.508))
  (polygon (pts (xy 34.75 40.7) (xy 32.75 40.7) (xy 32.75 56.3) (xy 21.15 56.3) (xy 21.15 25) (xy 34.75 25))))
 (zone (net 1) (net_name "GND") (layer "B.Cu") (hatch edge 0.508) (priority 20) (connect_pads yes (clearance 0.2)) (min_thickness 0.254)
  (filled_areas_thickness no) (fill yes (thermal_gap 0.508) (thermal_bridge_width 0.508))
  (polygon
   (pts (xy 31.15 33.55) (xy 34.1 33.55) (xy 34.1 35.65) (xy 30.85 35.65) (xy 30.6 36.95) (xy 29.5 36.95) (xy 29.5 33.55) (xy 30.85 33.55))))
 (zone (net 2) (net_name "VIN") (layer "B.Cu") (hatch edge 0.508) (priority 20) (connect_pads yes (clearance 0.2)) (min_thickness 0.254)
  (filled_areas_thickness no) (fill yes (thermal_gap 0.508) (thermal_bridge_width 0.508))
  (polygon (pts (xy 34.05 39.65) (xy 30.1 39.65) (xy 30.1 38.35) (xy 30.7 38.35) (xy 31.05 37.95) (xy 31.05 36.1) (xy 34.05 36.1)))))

